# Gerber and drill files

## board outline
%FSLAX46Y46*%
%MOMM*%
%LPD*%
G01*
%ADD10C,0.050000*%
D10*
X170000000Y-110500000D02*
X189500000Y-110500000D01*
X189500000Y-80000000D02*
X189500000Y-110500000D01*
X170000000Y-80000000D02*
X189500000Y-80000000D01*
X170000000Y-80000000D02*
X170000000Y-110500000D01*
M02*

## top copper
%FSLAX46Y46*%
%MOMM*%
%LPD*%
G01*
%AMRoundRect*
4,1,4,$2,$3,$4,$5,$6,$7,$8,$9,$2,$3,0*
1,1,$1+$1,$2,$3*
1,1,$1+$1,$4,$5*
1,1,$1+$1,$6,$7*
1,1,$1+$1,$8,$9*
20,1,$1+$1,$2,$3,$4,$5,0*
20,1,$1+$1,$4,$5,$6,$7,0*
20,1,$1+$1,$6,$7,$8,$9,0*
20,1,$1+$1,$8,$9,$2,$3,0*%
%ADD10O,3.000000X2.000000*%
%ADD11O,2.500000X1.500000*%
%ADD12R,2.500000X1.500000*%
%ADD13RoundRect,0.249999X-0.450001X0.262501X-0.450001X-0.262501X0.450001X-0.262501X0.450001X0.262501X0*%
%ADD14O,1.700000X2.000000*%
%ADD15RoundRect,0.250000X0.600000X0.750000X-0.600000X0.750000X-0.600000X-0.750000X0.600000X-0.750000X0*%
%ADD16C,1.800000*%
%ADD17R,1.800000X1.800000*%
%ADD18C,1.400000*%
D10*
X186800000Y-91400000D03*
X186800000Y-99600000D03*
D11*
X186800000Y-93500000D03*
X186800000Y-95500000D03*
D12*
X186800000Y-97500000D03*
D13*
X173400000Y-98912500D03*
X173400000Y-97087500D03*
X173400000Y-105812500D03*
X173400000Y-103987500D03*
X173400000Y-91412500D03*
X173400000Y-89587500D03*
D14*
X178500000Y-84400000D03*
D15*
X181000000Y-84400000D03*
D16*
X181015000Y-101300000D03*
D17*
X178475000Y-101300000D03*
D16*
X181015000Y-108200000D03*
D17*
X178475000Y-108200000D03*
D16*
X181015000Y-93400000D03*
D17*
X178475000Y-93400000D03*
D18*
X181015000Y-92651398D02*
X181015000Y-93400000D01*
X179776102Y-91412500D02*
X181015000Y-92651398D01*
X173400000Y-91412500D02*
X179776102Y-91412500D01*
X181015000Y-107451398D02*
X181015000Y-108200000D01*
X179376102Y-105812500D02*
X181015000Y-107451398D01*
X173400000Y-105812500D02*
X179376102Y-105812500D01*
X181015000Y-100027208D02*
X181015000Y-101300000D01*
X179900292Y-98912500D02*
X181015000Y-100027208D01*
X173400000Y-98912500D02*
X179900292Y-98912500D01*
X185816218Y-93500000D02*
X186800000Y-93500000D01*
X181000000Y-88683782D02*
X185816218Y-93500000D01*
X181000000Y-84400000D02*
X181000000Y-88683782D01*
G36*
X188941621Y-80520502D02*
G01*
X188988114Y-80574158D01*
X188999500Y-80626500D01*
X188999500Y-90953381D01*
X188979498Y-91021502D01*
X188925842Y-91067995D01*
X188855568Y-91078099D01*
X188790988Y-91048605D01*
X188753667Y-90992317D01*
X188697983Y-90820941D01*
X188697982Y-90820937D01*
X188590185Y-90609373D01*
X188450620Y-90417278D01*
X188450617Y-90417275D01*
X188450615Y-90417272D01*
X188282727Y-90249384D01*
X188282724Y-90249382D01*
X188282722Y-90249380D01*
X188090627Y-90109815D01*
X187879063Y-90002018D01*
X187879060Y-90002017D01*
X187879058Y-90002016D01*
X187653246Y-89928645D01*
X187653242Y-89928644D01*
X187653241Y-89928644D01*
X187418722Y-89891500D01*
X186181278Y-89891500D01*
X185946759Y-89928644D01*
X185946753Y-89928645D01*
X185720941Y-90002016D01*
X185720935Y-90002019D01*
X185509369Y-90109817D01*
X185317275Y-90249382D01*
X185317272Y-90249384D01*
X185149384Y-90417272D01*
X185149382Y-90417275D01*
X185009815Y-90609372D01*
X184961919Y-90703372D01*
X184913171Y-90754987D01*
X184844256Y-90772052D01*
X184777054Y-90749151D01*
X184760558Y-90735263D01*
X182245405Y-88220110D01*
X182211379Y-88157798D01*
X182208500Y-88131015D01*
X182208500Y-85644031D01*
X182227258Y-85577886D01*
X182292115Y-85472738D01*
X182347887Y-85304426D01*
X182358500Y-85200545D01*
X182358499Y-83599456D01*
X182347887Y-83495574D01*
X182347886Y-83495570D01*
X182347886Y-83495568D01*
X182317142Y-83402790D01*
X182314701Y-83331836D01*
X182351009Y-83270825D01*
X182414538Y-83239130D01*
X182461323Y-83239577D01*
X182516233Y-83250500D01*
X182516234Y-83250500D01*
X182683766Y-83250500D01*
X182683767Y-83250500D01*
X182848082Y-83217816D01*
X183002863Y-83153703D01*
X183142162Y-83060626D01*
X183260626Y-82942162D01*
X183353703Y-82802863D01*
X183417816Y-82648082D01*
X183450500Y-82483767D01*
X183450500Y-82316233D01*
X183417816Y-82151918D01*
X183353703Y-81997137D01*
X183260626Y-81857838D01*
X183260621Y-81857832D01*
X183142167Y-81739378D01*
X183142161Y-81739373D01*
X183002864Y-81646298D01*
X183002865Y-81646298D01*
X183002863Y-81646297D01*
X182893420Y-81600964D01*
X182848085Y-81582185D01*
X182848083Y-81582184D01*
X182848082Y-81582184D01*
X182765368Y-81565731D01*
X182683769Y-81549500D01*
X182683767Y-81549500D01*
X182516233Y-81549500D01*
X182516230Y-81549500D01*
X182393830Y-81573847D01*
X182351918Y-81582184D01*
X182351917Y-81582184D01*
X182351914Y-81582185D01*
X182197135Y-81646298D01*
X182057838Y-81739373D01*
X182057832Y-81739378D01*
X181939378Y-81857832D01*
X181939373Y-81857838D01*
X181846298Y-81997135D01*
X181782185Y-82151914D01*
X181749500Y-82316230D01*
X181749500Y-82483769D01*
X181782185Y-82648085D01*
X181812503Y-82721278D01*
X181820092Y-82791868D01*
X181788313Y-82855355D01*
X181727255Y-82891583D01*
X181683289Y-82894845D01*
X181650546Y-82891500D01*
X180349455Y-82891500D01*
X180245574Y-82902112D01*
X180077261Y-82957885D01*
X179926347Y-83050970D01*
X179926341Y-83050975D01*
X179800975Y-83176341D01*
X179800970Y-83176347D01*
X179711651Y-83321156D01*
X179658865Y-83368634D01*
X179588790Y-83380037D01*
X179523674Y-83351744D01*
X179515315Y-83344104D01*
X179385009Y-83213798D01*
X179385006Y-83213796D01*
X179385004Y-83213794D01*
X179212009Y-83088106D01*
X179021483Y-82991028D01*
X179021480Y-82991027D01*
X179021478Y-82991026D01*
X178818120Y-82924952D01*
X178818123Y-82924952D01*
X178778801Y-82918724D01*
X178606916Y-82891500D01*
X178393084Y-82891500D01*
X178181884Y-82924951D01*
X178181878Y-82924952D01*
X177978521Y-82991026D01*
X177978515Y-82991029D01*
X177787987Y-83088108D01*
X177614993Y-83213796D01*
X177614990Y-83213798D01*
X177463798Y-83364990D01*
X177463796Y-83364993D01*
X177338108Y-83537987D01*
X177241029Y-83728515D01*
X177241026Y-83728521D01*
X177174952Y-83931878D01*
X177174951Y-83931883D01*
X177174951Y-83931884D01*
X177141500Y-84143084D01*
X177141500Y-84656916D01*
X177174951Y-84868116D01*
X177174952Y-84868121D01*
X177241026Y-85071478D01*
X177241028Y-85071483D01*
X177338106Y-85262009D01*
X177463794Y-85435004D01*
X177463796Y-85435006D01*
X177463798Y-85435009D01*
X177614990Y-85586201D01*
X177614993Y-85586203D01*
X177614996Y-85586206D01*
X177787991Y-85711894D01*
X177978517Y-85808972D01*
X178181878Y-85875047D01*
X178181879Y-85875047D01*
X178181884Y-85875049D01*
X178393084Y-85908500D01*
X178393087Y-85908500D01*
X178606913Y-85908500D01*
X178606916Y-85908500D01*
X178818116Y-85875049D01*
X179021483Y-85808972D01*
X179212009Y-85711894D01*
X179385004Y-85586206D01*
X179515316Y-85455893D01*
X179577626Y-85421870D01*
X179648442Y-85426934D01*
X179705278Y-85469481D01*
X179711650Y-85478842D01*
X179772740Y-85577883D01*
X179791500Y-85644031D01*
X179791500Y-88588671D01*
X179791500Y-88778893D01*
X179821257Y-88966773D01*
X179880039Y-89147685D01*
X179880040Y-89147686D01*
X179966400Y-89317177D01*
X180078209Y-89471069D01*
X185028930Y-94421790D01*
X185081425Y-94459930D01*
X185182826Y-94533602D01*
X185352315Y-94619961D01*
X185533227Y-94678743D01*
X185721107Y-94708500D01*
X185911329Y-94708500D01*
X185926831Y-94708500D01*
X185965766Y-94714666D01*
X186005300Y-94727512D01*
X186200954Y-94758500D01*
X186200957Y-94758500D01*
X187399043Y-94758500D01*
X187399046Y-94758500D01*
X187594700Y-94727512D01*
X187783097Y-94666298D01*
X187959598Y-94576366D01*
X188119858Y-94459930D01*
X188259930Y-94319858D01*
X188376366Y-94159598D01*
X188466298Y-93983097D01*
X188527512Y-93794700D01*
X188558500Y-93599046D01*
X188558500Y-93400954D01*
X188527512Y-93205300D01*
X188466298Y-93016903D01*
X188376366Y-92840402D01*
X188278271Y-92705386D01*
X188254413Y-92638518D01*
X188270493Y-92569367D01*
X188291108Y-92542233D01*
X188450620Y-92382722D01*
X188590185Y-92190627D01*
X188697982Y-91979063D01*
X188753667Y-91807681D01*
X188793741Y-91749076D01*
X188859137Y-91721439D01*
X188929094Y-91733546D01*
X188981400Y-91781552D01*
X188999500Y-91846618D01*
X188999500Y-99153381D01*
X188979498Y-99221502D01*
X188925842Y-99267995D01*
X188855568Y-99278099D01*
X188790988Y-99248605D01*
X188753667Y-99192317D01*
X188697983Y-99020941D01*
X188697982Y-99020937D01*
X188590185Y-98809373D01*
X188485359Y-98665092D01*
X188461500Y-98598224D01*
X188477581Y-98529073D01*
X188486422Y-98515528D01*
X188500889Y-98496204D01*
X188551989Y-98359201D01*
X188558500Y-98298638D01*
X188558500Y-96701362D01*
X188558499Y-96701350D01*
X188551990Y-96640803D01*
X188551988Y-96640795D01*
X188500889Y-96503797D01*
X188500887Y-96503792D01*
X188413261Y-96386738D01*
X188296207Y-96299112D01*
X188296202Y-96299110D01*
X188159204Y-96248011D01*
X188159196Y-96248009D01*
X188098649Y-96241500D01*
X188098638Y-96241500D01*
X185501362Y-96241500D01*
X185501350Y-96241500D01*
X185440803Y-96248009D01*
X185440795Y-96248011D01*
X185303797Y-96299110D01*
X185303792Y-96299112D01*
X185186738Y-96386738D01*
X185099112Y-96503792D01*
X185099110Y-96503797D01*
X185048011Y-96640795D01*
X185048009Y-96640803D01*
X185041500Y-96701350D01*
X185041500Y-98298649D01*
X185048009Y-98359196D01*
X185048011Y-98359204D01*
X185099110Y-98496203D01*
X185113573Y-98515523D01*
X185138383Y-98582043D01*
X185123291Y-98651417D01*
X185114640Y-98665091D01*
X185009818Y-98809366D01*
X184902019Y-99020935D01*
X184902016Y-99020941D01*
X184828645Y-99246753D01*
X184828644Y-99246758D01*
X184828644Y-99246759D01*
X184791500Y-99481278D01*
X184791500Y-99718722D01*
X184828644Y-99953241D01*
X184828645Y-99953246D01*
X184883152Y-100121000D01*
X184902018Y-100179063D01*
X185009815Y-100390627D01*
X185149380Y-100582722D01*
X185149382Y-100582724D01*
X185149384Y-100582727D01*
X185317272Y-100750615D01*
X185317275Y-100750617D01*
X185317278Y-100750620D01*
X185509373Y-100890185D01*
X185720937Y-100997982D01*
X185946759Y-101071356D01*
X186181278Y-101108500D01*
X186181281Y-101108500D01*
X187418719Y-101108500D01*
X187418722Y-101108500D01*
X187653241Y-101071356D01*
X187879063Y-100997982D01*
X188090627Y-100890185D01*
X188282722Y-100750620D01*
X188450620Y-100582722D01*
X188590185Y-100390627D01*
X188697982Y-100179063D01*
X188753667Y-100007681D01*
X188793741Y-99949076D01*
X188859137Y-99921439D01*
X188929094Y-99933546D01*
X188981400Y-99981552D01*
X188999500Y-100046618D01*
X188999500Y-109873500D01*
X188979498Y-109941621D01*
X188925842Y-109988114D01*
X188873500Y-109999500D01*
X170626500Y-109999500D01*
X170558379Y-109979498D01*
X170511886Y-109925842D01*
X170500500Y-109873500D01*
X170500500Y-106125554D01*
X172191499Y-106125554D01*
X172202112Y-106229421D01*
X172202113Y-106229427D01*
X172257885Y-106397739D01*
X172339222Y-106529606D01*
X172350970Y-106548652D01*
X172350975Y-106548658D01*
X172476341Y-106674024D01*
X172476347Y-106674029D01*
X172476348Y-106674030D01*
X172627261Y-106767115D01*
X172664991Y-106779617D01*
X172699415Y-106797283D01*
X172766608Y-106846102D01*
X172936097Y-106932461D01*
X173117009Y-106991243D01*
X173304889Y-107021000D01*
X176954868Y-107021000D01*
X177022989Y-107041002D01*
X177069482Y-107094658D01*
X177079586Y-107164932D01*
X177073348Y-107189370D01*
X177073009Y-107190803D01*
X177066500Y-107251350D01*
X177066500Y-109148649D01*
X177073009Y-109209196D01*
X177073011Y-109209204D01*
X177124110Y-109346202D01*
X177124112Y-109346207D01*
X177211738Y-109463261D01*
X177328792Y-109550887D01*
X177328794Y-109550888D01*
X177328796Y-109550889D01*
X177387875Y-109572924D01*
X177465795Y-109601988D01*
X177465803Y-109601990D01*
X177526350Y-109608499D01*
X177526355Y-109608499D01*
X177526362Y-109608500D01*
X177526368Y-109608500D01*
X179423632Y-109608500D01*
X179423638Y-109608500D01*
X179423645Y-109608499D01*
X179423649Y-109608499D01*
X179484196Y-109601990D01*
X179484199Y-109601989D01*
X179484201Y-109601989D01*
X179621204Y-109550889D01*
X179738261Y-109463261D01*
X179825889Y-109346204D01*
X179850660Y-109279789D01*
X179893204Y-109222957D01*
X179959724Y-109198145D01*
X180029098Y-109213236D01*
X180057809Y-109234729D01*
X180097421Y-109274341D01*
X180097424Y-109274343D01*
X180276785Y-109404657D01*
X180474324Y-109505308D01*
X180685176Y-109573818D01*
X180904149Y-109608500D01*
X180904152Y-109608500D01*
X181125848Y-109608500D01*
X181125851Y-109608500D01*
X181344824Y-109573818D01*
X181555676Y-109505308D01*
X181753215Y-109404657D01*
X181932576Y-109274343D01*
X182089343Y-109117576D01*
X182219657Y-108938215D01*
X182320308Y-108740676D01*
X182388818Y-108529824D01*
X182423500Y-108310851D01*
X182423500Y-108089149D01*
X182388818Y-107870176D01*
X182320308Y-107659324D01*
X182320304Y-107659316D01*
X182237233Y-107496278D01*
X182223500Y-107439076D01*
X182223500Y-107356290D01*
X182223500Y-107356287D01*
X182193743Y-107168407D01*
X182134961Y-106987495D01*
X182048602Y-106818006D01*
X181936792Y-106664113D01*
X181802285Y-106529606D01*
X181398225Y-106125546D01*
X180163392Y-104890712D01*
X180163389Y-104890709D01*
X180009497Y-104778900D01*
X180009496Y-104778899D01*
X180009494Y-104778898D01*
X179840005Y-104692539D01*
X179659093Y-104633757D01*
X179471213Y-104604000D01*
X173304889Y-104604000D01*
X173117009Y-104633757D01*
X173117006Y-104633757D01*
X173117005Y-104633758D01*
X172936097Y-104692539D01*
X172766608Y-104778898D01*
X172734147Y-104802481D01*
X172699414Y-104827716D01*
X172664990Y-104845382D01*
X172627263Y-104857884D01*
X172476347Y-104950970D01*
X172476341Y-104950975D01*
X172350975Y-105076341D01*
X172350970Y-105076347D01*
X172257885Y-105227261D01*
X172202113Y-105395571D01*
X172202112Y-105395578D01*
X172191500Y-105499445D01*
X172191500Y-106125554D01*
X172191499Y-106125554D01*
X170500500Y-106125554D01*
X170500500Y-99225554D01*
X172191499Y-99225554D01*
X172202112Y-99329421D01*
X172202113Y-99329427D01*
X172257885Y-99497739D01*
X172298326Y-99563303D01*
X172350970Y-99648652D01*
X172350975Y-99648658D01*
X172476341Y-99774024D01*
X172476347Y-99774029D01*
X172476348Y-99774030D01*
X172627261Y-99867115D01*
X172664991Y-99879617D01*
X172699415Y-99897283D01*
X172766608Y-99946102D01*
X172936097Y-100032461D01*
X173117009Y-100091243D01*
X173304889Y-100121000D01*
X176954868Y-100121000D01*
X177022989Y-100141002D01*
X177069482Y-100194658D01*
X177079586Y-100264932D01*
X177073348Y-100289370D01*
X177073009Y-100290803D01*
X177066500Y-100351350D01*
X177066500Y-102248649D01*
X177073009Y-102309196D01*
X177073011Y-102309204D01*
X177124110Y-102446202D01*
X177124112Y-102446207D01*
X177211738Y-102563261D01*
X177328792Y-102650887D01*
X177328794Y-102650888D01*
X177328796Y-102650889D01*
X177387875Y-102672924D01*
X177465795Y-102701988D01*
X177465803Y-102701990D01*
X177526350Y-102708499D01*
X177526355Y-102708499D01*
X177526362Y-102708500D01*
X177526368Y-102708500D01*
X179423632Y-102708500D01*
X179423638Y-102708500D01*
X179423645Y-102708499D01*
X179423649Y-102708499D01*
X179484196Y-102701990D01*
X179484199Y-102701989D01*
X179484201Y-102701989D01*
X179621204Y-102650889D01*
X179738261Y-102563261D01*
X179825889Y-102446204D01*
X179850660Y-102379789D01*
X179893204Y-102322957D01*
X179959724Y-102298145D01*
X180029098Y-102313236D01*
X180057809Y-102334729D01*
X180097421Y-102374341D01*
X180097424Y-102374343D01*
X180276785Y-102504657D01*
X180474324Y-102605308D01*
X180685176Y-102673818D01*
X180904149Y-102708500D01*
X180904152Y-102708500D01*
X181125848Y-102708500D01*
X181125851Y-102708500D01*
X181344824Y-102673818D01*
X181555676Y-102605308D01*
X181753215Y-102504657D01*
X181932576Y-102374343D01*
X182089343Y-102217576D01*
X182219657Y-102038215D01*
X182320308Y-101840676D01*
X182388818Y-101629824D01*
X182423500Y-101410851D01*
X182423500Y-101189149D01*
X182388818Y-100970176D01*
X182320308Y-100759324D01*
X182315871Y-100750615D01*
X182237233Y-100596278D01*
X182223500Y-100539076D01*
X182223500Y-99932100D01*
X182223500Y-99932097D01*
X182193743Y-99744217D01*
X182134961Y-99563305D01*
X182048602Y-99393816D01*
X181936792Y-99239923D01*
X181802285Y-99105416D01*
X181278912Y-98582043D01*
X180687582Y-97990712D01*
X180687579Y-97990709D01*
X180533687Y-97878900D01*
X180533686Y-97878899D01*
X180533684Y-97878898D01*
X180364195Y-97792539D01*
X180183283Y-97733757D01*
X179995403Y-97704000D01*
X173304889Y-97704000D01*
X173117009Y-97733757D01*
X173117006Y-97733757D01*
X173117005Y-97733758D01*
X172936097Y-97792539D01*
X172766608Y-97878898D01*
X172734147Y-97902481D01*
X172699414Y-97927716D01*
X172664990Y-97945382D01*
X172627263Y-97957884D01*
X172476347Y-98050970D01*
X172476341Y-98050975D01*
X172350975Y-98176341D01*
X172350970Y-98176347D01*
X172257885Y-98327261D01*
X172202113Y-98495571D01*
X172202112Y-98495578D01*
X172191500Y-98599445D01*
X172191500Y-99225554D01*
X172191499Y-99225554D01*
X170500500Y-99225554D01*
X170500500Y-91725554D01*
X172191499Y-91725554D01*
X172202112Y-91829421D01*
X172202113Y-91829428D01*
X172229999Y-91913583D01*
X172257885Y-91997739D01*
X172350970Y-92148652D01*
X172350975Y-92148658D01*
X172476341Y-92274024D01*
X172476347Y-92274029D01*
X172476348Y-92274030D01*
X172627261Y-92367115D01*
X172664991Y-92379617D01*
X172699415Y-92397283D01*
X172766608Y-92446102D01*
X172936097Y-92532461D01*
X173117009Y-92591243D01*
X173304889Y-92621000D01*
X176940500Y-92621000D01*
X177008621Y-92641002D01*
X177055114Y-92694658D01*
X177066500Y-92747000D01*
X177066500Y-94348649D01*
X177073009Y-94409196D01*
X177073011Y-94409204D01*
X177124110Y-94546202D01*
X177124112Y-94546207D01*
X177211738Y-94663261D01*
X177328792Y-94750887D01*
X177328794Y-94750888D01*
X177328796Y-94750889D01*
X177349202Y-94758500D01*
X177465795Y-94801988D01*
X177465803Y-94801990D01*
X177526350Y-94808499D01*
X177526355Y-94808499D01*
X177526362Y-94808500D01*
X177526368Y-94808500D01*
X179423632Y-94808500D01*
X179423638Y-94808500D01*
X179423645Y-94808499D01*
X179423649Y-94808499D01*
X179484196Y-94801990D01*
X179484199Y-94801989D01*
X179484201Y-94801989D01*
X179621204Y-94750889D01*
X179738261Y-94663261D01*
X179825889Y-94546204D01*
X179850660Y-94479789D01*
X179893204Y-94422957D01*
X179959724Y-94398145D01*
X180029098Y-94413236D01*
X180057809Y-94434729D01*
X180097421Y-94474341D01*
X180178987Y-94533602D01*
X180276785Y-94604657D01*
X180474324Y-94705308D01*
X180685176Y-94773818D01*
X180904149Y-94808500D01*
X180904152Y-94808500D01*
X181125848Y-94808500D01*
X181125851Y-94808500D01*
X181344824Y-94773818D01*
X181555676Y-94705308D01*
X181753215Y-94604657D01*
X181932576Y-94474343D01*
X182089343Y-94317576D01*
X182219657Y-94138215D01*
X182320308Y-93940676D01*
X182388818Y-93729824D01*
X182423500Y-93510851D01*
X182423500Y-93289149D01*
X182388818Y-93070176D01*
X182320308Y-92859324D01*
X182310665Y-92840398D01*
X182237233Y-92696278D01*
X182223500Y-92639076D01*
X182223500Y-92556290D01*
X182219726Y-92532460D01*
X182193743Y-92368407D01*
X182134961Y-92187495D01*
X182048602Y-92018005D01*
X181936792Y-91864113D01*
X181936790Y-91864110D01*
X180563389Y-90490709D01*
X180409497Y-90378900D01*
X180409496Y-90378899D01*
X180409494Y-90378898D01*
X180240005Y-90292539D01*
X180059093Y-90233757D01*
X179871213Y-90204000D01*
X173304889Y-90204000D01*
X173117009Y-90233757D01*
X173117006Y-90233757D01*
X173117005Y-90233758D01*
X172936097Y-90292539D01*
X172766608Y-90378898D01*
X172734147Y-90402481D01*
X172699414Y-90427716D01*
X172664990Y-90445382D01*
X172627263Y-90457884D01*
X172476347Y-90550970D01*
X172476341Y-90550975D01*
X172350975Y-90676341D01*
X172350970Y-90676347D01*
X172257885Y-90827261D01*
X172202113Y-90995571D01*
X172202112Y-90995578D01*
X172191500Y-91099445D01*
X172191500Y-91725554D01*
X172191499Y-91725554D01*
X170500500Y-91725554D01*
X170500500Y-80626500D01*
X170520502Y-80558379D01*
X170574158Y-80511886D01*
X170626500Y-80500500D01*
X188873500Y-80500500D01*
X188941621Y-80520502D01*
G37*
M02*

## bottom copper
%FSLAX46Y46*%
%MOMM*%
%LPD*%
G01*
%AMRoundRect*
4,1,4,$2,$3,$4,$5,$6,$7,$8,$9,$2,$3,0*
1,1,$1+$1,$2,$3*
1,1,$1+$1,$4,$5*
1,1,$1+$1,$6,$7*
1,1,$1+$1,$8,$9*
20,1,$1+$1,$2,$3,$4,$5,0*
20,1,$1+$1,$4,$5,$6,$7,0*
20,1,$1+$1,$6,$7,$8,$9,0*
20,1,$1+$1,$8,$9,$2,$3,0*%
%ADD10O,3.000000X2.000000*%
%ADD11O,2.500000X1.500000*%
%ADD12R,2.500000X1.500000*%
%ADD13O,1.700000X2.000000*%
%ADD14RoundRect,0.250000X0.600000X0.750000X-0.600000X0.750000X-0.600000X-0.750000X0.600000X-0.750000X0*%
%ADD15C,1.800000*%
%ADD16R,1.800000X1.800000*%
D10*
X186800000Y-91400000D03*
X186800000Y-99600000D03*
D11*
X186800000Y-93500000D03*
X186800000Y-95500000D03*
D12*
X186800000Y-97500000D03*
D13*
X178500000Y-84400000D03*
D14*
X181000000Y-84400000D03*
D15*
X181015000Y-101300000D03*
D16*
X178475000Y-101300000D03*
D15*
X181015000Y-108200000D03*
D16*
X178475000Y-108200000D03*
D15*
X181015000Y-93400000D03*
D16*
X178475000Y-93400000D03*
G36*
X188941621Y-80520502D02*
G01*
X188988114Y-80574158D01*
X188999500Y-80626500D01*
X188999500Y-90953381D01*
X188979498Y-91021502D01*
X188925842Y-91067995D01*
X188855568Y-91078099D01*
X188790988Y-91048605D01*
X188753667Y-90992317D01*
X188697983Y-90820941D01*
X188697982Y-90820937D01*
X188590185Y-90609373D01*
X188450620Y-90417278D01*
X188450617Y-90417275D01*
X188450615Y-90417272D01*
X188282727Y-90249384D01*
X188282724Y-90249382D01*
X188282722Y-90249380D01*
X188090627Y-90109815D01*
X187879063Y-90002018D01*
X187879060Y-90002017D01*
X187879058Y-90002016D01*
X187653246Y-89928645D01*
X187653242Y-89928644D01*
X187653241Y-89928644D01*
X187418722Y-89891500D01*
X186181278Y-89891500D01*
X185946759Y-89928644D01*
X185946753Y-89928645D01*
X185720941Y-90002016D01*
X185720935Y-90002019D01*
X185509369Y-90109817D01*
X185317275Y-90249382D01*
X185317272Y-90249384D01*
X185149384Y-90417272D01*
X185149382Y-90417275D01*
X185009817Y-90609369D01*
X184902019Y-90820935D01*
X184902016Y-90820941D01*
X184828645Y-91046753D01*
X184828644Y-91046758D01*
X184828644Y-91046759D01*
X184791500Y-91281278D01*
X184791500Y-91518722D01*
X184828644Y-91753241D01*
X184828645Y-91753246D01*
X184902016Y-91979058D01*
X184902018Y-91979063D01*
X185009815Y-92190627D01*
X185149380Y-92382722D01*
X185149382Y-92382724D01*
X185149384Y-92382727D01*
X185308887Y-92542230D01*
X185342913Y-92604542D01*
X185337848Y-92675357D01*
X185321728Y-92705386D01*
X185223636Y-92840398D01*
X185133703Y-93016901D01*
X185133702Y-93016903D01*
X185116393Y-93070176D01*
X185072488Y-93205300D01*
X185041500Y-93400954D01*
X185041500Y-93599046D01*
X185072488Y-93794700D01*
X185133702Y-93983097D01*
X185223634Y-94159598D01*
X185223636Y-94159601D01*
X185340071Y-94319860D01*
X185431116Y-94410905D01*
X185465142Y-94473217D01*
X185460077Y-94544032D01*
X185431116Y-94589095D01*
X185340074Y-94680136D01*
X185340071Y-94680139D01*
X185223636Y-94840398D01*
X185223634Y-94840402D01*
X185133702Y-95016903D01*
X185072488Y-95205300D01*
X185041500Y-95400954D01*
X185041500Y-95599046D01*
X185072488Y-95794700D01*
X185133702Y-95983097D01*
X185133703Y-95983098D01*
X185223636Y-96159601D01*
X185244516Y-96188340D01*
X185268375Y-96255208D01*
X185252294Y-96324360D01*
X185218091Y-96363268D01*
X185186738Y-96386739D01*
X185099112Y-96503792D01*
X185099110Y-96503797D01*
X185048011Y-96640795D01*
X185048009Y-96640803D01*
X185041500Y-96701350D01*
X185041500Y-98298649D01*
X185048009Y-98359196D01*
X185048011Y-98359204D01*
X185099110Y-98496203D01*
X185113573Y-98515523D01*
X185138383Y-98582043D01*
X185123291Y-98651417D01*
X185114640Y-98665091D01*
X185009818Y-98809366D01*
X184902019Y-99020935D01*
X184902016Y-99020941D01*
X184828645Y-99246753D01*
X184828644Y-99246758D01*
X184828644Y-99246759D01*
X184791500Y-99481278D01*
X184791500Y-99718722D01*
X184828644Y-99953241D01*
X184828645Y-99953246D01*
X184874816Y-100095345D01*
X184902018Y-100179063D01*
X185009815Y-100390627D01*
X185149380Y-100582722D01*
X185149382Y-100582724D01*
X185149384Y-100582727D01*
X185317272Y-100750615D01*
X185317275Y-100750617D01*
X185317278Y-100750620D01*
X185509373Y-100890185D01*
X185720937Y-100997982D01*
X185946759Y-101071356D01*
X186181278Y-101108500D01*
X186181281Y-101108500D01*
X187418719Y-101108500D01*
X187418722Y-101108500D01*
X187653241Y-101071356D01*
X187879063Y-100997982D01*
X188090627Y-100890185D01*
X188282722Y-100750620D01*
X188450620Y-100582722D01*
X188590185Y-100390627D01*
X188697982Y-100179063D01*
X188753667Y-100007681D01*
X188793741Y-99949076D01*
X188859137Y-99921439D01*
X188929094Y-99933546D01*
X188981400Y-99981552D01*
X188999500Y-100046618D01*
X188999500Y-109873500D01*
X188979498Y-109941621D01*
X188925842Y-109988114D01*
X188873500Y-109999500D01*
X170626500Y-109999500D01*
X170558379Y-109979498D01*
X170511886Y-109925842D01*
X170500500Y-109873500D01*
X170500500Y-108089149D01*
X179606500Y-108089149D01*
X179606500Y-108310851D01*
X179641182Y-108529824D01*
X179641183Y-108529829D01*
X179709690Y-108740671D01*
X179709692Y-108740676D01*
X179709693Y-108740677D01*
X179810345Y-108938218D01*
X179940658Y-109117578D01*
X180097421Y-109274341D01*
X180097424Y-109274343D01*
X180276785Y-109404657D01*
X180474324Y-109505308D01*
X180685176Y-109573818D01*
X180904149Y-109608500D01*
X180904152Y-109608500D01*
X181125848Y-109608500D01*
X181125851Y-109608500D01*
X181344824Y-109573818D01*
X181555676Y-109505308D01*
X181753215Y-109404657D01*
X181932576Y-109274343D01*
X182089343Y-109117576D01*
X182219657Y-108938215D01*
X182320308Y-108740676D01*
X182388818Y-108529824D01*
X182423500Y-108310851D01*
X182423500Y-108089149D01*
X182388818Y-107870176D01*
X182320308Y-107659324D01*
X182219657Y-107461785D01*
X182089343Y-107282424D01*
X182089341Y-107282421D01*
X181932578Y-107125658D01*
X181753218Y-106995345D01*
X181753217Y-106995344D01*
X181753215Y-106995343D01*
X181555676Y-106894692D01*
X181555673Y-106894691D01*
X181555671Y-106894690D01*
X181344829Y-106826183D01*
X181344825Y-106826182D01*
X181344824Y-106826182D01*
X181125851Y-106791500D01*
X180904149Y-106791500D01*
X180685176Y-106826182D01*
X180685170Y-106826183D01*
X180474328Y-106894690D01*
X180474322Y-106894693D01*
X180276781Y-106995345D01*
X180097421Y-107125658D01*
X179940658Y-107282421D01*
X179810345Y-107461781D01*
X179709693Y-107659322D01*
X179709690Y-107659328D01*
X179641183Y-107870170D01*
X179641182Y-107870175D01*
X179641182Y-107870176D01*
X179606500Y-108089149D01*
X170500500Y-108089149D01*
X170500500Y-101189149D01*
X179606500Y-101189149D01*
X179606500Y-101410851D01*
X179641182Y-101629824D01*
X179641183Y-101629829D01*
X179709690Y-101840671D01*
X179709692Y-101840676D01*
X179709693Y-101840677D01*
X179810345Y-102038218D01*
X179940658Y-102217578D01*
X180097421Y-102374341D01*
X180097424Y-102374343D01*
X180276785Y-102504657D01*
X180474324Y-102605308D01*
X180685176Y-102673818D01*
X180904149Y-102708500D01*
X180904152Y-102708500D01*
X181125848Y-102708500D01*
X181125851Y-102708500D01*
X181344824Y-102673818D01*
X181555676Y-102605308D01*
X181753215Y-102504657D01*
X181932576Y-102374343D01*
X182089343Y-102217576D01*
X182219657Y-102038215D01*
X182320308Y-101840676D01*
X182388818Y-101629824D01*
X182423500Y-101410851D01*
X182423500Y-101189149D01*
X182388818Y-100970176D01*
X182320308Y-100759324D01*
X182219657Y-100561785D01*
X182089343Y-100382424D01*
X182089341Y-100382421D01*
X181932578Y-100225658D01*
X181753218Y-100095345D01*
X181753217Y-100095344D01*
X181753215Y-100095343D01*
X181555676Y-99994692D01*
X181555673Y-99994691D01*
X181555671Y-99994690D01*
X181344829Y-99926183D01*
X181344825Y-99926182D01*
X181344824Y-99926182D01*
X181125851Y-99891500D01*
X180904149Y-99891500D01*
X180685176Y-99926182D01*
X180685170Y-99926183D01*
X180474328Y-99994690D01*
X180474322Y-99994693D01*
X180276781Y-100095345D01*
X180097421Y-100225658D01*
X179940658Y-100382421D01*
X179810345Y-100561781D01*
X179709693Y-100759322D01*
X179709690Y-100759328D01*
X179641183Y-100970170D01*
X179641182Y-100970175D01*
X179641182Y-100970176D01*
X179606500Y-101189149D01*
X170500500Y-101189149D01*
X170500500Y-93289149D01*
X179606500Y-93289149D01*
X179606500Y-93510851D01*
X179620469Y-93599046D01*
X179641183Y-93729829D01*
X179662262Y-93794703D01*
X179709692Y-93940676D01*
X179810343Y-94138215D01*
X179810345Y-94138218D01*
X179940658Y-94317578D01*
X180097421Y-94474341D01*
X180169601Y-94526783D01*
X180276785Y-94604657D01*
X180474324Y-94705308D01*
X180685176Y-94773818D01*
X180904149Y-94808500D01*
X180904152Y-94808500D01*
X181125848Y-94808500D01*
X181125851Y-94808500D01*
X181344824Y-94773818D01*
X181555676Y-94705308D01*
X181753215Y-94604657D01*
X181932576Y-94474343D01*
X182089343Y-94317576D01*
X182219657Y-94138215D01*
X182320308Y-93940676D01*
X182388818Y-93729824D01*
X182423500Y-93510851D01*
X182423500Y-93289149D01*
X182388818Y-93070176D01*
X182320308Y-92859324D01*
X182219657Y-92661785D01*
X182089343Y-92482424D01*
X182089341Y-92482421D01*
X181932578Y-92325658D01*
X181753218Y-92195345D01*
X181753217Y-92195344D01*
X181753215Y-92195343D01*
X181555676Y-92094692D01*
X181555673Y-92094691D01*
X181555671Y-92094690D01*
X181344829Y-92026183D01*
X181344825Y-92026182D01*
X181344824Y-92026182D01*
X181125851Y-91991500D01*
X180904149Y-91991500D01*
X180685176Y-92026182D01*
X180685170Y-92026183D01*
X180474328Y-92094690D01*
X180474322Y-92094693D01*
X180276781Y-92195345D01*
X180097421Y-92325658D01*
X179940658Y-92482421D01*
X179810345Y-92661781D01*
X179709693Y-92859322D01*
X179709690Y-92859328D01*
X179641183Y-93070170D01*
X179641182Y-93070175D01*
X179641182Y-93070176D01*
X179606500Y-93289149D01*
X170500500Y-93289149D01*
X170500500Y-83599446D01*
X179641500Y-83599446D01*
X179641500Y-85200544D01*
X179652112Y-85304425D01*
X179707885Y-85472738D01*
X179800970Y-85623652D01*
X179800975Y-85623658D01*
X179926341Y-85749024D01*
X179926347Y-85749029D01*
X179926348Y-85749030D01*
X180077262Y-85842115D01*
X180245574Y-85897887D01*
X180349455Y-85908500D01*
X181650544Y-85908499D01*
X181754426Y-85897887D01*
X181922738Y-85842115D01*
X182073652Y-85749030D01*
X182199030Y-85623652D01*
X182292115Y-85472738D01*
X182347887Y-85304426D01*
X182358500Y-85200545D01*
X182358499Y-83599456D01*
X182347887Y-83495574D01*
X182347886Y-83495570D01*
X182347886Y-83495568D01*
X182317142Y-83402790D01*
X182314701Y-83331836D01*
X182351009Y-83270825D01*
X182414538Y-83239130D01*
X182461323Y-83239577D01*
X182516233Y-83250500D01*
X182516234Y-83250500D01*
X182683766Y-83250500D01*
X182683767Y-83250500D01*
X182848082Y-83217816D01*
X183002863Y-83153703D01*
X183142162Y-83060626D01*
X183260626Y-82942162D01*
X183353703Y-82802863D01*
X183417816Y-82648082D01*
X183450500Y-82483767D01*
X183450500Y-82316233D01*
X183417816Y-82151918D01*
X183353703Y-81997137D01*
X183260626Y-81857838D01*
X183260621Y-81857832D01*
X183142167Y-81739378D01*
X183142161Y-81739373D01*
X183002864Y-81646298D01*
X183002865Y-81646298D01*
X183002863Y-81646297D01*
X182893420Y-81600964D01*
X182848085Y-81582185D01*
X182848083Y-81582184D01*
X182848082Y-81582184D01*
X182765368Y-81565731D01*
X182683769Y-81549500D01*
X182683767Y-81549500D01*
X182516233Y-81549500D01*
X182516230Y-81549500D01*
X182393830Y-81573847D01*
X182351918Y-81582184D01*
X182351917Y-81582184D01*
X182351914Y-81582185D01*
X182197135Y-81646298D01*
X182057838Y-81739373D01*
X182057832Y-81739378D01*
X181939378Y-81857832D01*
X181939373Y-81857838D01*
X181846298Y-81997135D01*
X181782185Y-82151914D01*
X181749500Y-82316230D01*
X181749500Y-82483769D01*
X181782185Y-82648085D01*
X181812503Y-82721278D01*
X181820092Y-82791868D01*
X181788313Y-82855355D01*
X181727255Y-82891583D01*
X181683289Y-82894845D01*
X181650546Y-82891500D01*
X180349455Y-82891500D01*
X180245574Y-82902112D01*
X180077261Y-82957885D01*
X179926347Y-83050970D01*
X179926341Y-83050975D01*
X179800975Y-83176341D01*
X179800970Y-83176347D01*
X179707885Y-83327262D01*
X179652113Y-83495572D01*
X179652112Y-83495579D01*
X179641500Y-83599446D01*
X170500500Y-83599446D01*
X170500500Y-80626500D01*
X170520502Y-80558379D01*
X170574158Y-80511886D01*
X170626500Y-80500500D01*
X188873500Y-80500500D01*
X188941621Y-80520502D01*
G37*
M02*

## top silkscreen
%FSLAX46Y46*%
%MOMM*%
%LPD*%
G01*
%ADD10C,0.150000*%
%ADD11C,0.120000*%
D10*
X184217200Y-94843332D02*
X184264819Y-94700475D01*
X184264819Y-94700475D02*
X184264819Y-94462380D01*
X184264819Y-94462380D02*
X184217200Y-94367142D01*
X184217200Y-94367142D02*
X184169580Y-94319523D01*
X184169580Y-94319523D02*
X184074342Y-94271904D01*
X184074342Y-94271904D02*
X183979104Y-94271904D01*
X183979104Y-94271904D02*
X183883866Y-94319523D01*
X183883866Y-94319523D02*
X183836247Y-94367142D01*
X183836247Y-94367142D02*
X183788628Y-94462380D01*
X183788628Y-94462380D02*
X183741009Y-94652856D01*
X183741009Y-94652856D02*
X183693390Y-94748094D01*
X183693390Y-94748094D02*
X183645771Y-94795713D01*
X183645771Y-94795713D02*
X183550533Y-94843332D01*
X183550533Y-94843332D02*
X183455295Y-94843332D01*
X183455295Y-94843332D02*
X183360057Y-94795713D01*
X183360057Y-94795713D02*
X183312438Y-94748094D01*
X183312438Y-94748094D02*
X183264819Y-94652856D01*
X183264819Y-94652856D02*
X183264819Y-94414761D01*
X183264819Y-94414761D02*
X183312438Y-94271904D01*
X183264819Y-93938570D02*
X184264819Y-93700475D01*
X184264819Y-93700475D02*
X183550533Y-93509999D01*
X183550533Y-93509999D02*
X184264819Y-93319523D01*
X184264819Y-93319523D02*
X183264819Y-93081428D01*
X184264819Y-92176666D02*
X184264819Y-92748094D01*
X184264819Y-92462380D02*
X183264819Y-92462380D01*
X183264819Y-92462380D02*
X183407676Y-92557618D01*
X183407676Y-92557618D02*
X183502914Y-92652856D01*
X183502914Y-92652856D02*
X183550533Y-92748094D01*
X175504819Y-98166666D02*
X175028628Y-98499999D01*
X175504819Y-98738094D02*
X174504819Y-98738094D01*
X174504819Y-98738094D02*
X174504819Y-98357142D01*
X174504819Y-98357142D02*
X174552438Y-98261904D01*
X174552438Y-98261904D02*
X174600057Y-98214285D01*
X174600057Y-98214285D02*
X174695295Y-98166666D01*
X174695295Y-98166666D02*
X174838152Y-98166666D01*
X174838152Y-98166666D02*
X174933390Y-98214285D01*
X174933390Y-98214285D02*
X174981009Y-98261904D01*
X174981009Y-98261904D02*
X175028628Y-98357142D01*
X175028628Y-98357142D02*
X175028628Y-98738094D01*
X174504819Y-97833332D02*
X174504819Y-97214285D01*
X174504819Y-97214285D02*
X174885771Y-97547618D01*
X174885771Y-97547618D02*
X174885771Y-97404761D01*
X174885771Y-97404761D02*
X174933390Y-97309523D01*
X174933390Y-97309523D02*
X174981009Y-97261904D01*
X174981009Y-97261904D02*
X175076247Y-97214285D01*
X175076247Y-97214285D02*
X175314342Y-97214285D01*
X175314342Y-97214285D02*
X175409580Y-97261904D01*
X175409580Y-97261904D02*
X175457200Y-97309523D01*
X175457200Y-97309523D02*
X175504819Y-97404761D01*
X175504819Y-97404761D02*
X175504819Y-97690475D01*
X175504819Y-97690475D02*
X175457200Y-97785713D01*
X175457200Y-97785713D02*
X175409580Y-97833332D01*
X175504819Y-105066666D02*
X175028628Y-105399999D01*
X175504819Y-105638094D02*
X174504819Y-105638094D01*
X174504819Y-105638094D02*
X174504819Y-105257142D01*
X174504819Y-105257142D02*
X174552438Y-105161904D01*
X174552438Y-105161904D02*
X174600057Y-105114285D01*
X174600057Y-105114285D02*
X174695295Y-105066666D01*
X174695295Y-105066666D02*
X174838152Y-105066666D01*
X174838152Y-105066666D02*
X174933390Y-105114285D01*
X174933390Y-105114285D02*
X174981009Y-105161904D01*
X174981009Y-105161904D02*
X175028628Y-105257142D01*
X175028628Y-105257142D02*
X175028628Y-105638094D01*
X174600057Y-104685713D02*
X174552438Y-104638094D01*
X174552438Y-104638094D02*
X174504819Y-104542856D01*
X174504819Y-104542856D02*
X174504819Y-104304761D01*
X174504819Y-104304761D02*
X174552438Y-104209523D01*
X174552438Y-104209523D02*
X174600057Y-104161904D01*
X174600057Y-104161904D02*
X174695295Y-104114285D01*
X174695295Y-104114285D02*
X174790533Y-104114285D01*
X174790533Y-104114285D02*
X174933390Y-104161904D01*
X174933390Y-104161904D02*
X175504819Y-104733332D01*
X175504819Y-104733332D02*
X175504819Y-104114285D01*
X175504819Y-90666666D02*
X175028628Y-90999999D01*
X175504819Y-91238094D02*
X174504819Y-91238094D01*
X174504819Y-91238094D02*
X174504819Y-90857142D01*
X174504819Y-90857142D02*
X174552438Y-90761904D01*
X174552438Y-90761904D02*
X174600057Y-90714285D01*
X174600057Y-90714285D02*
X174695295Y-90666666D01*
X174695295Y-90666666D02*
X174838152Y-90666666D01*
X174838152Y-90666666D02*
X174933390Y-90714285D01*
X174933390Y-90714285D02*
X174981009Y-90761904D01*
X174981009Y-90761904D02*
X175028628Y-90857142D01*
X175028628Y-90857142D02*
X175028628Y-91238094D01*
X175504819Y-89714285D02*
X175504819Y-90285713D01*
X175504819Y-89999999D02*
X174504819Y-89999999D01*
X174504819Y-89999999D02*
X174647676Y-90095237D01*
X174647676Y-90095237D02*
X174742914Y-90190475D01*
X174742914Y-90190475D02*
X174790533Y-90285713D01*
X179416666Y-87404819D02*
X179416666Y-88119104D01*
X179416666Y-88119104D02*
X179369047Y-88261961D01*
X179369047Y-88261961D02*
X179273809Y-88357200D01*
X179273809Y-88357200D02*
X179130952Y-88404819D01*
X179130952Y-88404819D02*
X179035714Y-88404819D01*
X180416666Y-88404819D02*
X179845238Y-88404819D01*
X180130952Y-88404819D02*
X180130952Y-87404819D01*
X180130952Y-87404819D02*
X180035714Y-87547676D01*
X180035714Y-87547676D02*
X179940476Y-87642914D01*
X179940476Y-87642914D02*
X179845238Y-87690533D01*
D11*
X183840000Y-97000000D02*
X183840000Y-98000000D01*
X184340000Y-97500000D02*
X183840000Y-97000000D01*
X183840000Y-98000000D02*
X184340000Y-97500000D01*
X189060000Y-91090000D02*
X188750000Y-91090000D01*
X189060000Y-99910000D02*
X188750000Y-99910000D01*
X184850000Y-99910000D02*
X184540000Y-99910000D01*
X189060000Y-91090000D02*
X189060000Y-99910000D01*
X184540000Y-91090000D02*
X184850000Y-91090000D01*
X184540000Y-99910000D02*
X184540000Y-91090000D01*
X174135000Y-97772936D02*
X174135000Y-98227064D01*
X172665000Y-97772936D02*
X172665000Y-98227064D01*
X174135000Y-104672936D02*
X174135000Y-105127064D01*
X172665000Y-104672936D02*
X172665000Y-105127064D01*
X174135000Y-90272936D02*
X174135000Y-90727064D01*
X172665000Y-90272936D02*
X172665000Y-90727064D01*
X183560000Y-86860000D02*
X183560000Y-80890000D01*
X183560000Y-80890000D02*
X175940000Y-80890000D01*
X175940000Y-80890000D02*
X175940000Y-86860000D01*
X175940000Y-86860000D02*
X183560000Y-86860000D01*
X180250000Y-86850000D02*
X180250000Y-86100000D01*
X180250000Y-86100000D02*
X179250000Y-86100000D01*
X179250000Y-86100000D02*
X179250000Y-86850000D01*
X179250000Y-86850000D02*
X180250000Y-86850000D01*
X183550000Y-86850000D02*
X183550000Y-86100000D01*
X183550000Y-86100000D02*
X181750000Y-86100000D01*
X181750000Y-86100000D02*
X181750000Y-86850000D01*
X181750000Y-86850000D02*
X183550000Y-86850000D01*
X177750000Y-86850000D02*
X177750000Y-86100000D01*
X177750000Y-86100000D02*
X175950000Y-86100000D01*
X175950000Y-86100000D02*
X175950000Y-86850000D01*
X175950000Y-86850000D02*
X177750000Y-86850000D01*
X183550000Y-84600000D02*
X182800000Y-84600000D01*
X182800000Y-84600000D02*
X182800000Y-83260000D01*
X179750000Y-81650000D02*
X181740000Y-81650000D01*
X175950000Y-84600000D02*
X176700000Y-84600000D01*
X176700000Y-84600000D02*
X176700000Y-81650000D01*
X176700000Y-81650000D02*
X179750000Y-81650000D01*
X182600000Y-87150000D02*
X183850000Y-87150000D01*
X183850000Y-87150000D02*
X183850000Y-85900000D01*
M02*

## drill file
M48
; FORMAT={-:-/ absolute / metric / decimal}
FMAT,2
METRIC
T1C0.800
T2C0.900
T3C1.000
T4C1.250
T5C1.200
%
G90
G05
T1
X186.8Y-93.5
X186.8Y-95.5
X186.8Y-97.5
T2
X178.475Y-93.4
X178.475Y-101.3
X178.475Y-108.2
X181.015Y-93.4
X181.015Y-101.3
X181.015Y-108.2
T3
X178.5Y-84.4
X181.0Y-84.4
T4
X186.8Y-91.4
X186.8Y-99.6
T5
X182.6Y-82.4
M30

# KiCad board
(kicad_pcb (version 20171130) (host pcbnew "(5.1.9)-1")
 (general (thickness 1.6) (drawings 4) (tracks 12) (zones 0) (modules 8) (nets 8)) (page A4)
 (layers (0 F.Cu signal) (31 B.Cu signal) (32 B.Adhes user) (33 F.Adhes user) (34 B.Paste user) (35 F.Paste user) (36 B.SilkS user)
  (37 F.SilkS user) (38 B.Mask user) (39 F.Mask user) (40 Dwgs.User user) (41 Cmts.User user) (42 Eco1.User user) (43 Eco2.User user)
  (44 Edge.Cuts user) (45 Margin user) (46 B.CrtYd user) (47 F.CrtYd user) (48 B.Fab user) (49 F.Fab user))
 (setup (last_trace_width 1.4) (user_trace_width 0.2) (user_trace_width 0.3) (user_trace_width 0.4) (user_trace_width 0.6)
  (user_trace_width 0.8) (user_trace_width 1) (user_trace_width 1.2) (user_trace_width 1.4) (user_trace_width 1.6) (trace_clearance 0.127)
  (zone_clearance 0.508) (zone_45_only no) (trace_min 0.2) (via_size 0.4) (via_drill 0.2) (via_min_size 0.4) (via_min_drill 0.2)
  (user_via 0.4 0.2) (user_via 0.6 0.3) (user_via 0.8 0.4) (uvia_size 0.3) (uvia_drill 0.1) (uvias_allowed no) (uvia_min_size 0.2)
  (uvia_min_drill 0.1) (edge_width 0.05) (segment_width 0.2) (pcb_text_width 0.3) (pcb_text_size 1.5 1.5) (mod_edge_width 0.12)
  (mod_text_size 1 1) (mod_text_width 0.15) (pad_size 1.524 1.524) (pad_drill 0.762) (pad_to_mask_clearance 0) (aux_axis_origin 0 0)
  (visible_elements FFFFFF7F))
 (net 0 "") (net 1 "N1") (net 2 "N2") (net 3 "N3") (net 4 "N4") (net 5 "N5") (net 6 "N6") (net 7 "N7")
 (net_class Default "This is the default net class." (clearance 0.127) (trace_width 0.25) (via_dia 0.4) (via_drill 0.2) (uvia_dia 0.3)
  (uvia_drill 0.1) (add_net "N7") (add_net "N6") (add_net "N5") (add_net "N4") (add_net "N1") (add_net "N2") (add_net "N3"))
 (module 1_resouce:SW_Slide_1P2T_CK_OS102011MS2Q (layer F.Cu) (at 186.8 97.5 90)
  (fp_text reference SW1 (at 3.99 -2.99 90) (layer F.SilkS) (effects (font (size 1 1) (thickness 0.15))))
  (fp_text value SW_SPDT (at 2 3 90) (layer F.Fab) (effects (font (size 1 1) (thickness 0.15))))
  (fp_line (start 0.5 -2.96) (end -0.5 -2.96) (layer F.SilkS) (width 0.12))
  (fp_line (start 0 -2.46) (end 0.5 -2.96) (layer F.SilkS) (width 0.12))
  (fp_line (start -0.5 -2.96) (end 0 -2.46) (layer F.SilkS) (width 0.12))
  (fp_line (start 6.41 2.26) (end 6.41 1.95) (layer F.SilkS) (width 0.12))
  (fp_line (start -2.41 2.26) (end -2.41 1.95) (layer F.SilkS) (width 0.12))
  (fp_line (start -2.41 -1.95) (end -2.41 -2.26) (layer F.SilkS) (width 0.12))
  (fp_line (start 6.41 2.26) (end -2.41 2.26) (layer F.SilkS) (width 0.12))
  (fp_line (start 6.41 -2.26) (end 6.41 -1.95) (layer F.SilkS) (width 0.12))
  (fp_line (start -2.41 -2.26) (end 6.41 -2.26) (layer F.SilkS) (width 0.12))
  (pad "" thru_hole oval (at 6.1 0 90) (size 2 3) (drill 1.25) (layers *.Cu *.Mask))
  (pad "" thru_hole oval (at -2.1 0 90) (size 2 3) (drill 1.25) (layers *.Cu *.Mask))
  (pad 3 thru_hole oval (at 4 0 90) (size 1.5 2.5) (drill 0.8) (layers *.Cu *.Mask) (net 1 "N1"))
  (pad 2 thru_hole oval (at 2 0 90) (size 1.5 2.5) (drill 0.8) (layers *.Cu *.Mask) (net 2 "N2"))
  (pad 1 thru_hole rect (at 0 0 90) (size 1.5 2.5) (drill 0.8) (layers *.Cu *.Mask) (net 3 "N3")))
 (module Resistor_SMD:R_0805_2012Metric (layer F.Cu) (at 173.4 98 270)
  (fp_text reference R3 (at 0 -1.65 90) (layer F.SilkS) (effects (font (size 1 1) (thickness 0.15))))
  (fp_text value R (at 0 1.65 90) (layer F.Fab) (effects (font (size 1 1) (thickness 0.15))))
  (fp_line (start -0.227064 -0.735) (end 0.227064 -0.735) (layer F.SilkS) (width 0.12))
  (fp_line (start -0.227064 0.735) (end 0.227064 0.735) (layer F.SilkS) (width 0.12))
  (pad 2 smd roundrect (at 0.9125 0 270) (size 1.025 1.4) (layers F.Cu F.Paste F.Mask) (roundrect_rratio 0.2439014634146341) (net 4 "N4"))
  (pad 1 smd roundrect (at -0.9125 0 270) (size 1.025 1.4) (layers F.Cu F.Paste F.Mask) (roundrect_rratio 0.2439014634146341) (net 2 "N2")))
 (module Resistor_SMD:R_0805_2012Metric (layer F.Cu) (at 173.4 104.9 270)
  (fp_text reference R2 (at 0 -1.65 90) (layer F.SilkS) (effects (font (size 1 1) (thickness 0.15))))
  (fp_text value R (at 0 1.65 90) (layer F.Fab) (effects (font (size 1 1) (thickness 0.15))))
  (fp_line (start -0.227064 -0.735) (end 0.227064 -0.735) (layer F.SilkS) (width 0.12))
  (fp_line (start -0.227064 0.735) (end 0.227064 0.735) (layer F.SilkS) (width 0.12))
  (pad 2 smd roundrect (at 0.9125 0 270) (size 1.025 1.4) (layers F.Cu F.Paste F.Mask) (roundrect_rratio 0.2439014634146341) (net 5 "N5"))
  (pad 1 smd roundrect (at -0.9125 0 270) (size 1.025 1.4) (layers F.Cu F.Paste F.Mask) (roundrect_rratio 0.2439014634146341) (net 2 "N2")))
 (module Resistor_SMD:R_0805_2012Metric (layer F.Cu) (at 173.4 90.5 270)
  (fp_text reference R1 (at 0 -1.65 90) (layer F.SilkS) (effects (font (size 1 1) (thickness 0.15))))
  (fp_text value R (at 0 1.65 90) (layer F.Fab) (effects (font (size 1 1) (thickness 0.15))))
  (fp_line (start -0.227064 -0.735) (end 0.227064 -0.735) (layer F.SilkS) (width 0.12))
  (fp_line (start -0.227064 0.735) (end 0.227064 0.735) (layer F.SilkS) (width 0.12))
  (pad 2 smd roundrect (at 0.9125 0 270) (size 1.025 1.4) (layers F.Cu F.Paste F.Mask) (roundrect_rratio 0.2439014634146341) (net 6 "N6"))
  (pad 1 smd roundrect (at -0.9125 0 270) (size 1.025 1.4) (layers F.Cu F.Paste F.Mask) (roundrect_rratio 0.2439014634146341) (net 2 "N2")))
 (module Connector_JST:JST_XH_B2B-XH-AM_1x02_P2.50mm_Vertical (layer F.Cu) (at 181 84.4 180)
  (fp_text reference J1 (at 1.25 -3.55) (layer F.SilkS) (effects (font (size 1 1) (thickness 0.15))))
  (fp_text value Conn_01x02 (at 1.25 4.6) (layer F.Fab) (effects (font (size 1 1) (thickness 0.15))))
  (fp_line (start -2.56 -2.46) (end -2.56 3.51) (layer F.SilkS) (width 0.12))
  (fp_line (start -2.56 3.51) (end 5.06 3.51) (layer F.SilkS) (width 0.12))
  (fp_line (start 5.06 3.51) (end 5.06 -2.46) (layer F.SilkS) (width 0.12))
  (fp_line (start 5.06 -2.46) (end -2.56 -2.46) (layer F.SilkS) (width 0.12))
  (fp_line (start 0.75 -2.45) (end 0.75 -1.7) (layer F.SilkS) (width 0.12))
  (fp_line (start 0.75 -1.7) (end 1.75 -1.7) (layer F.SilkS) (width 0.12))
  (fp_line (start 1.75 -1.7) (end 1.75 -2.45) (layer F.SilkS) (width 0.12))
  (fp_line (start 1.75 -2.45) (end 0.75 -2.45) (layer F.SilkS) (width 0.12))
  (fp_line (start -2.55 -2.45) (end -2.55 -1.7) (layer F.SilkS) (width 0.12))
  (fp_line (start -2.55 -1.7) (end -0.75 -1.7) (layer F.SilkS) (width 0.12))
  (fp_line (start -0.75 -1.7) (end -0.75 -2.45) (layer F.SilkS) (width 0.12))
  (fp_line (start -0.75 -2.45) (end -2.55 -2.45) (layer F.SilkS) (width 0.12))
  (fp_line (start 3.25 -2.45) (end 3.25 -1.7) (layer F.SilkS) (width 0.12))
  (fp_line (start 3.25 -1.7) (end 5.05 -1.7) (layer F.SilkS) (width 0.12))
  (fp_line (start 5.05 -1.7) (end 5.05 -2.45) (layer F.SilkS) (width 0.12))
  (fp_line (start 5.05 -2.45) (end 3.25 -2.45) (layer F.SilkS) (width 0.12))
  (fp_line (start -2.55 -0.2) (end -1.8 -0.2) (layer F.SilkS) (width 0.12))
  (fp_line (start -1.8 -0.2) (end -1.8 1.14) (layer F.SilkS) (width 0.12))
  (fp_line (start 1.25 2.75) (end -0.74 2.75) (layer F.SilkS) (width 0.12))
  (fp_line (start 5.05 -0.2) (end 4.3 -0.2) (layer F.SilkS) (width 0.12))
  (fp_line (start 4.3 -0.2) (end 4.3 2.75) (layer F.SilkS) (width 0.12))
  (fp_line (start 4.3 2.75) (end 1.25 2.75) (layer F.SilkS) (width 0.12))
  (fp_line (start -1.6 -2.75) (end -2.85 -2.75) (layer F.SilkS) (width 0.12))
  (fp_line (start -2.85 -2.75) (end -2.85 -1.5) (layer F.SilkS) (width 0.12))
  (pad "" np_thru_hole circle (at -1.6 2 180) (size 1.2 1.2) (drill 1.2) (layers *.Cu *.Mask))
  (pad 2 thru_hole oval (at 2.5 0 180) (size 1.7 2) (drill 1) (layers *.Cu *.Mask) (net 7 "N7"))
  (pad 1 thru_hole roundrect (at 0 0 180) (size 1.7 2) (drill 1) (layers *.Cu *.Mask) (roundrect_rratio 0.1470588235294118) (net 1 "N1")))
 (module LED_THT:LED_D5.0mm (layer B.Cu) (at 178.475 101.3)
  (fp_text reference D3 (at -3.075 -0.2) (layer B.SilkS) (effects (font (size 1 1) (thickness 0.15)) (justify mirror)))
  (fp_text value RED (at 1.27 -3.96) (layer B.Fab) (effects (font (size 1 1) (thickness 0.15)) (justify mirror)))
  (pad 2 thru_hole circle (at 2.54 0) (size 1.8 1.8) (drill 0.9) (layers *.Cu *.Mask) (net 4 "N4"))
  (pad 1 thru_hole rect (at 0 0) (size 1.8 1.8) (drill 0.9) (layers *.Cu *.Mask) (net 7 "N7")))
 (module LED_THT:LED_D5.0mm (layer B.Cu) (at 178.475 108.2)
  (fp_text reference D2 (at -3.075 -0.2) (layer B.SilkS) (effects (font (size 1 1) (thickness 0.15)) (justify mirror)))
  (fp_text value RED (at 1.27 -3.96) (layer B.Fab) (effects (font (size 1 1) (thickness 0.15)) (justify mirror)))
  (pad 2 thru_hole circle (at 2.54 0) (size 1.8 1.8) (drill 0.9) (layers *.Cu *.Mask) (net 5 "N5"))
  (pad 1 thru_hole rect (at 0 0) (size 1.8 1.8) (drill 0.9) (layers *.Cu *.Mask) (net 7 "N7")))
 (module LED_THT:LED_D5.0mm (layer B.Cu) (at 178.475 93.4)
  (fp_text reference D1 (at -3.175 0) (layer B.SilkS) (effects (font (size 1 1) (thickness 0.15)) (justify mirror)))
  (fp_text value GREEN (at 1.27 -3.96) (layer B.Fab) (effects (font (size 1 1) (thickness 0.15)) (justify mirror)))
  (pad 2 thru_hole circle (at 2.54 0) (size 1.8 1.8) (drill 0.9) (layers *.Cu *.Mask) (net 6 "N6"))
  (pad 1 thru_hole rect (at 0 0) (size 1.8 1.8) (drill 0.9) (layers *.Cu *.Mask) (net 7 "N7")))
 (gr_line (start 170 110.5) (end 189.5 110.5) (layer Edge.Cuts) (width 0.05))
 (gr_line (start 189.5 80) (end 189.5 110.5) (layer Edge.Cuts) (width 0.05))
 (gr_line (start 170 80) (end 189.5 80) (layer Edge.Cuts) (width 0.05))
 (gr_line (start 170 80) (end 170 110.5) (layer Edge.Cuts) (width 0.05))
 (segment (start 181.015 92.651398) (end 181.015 93.4) (width 1.4) (layer F.Cu) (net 6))
 (segment (start 179.776102 91.4125) (end 181.015 92.651398) (width 1.4) (layer F.Cu) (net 6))
 (segment (start 173.4 91.4125) (end 179.776102 91.4125) (width 1.4) (layer F.Cu) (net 6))
 (segment (start 181.015 107.451398) (end 181.015 108.2) (width 1.4) (layer F.Cu) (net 5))
 (segment (start 179.376102 105.8125) (end 181.015 107.451398) (width 1.4) (layer F.Cu) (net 5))
 (segment (start 173.4 105.8125) (end 179.376102 105.8125) (width 1.4) (layer F.Cu) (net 5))
 (segment (start 181.015 100.027208) (end 181.015 101.3) (width 1.4) (layer F.Cu) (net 4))
 (segment (start 179.900292 98.9125) (end 181.015 100.027208) (width 1.4) (layer F.Cu) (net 4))
 (segment (start 173.4 98.9125) (end 179.900292 98.9125) (width 1.4) (layer F.Cu) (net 4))
 (segment (start 185.816218 93.5) (end 186.8 93.5) (width 1.4) (layer F.Cu) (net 1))
 (segment (start 181 88.683782) (end 185.816218 93.5) (width 1.4) (layer F.Cu) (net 1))
 (segment (start 181 84.4) (end 181 88.683782) (width 1.4) (layer F.Cu) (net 1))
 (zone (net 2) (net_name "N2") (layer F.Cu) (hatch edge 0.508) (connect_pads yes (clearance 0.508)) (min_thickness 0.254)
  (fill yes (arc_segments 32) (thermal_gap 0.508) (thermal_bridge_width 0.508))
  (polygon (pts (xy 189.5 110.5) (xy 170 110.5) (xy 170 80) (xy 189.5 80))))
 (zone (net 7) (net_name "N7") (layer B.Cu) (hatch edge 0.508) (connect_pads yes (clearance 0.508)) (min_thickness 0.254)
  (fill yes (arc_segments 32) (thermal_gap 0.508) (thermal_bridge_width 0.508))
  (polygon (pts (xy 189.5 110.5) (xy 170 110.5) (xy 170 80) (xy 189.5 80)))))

